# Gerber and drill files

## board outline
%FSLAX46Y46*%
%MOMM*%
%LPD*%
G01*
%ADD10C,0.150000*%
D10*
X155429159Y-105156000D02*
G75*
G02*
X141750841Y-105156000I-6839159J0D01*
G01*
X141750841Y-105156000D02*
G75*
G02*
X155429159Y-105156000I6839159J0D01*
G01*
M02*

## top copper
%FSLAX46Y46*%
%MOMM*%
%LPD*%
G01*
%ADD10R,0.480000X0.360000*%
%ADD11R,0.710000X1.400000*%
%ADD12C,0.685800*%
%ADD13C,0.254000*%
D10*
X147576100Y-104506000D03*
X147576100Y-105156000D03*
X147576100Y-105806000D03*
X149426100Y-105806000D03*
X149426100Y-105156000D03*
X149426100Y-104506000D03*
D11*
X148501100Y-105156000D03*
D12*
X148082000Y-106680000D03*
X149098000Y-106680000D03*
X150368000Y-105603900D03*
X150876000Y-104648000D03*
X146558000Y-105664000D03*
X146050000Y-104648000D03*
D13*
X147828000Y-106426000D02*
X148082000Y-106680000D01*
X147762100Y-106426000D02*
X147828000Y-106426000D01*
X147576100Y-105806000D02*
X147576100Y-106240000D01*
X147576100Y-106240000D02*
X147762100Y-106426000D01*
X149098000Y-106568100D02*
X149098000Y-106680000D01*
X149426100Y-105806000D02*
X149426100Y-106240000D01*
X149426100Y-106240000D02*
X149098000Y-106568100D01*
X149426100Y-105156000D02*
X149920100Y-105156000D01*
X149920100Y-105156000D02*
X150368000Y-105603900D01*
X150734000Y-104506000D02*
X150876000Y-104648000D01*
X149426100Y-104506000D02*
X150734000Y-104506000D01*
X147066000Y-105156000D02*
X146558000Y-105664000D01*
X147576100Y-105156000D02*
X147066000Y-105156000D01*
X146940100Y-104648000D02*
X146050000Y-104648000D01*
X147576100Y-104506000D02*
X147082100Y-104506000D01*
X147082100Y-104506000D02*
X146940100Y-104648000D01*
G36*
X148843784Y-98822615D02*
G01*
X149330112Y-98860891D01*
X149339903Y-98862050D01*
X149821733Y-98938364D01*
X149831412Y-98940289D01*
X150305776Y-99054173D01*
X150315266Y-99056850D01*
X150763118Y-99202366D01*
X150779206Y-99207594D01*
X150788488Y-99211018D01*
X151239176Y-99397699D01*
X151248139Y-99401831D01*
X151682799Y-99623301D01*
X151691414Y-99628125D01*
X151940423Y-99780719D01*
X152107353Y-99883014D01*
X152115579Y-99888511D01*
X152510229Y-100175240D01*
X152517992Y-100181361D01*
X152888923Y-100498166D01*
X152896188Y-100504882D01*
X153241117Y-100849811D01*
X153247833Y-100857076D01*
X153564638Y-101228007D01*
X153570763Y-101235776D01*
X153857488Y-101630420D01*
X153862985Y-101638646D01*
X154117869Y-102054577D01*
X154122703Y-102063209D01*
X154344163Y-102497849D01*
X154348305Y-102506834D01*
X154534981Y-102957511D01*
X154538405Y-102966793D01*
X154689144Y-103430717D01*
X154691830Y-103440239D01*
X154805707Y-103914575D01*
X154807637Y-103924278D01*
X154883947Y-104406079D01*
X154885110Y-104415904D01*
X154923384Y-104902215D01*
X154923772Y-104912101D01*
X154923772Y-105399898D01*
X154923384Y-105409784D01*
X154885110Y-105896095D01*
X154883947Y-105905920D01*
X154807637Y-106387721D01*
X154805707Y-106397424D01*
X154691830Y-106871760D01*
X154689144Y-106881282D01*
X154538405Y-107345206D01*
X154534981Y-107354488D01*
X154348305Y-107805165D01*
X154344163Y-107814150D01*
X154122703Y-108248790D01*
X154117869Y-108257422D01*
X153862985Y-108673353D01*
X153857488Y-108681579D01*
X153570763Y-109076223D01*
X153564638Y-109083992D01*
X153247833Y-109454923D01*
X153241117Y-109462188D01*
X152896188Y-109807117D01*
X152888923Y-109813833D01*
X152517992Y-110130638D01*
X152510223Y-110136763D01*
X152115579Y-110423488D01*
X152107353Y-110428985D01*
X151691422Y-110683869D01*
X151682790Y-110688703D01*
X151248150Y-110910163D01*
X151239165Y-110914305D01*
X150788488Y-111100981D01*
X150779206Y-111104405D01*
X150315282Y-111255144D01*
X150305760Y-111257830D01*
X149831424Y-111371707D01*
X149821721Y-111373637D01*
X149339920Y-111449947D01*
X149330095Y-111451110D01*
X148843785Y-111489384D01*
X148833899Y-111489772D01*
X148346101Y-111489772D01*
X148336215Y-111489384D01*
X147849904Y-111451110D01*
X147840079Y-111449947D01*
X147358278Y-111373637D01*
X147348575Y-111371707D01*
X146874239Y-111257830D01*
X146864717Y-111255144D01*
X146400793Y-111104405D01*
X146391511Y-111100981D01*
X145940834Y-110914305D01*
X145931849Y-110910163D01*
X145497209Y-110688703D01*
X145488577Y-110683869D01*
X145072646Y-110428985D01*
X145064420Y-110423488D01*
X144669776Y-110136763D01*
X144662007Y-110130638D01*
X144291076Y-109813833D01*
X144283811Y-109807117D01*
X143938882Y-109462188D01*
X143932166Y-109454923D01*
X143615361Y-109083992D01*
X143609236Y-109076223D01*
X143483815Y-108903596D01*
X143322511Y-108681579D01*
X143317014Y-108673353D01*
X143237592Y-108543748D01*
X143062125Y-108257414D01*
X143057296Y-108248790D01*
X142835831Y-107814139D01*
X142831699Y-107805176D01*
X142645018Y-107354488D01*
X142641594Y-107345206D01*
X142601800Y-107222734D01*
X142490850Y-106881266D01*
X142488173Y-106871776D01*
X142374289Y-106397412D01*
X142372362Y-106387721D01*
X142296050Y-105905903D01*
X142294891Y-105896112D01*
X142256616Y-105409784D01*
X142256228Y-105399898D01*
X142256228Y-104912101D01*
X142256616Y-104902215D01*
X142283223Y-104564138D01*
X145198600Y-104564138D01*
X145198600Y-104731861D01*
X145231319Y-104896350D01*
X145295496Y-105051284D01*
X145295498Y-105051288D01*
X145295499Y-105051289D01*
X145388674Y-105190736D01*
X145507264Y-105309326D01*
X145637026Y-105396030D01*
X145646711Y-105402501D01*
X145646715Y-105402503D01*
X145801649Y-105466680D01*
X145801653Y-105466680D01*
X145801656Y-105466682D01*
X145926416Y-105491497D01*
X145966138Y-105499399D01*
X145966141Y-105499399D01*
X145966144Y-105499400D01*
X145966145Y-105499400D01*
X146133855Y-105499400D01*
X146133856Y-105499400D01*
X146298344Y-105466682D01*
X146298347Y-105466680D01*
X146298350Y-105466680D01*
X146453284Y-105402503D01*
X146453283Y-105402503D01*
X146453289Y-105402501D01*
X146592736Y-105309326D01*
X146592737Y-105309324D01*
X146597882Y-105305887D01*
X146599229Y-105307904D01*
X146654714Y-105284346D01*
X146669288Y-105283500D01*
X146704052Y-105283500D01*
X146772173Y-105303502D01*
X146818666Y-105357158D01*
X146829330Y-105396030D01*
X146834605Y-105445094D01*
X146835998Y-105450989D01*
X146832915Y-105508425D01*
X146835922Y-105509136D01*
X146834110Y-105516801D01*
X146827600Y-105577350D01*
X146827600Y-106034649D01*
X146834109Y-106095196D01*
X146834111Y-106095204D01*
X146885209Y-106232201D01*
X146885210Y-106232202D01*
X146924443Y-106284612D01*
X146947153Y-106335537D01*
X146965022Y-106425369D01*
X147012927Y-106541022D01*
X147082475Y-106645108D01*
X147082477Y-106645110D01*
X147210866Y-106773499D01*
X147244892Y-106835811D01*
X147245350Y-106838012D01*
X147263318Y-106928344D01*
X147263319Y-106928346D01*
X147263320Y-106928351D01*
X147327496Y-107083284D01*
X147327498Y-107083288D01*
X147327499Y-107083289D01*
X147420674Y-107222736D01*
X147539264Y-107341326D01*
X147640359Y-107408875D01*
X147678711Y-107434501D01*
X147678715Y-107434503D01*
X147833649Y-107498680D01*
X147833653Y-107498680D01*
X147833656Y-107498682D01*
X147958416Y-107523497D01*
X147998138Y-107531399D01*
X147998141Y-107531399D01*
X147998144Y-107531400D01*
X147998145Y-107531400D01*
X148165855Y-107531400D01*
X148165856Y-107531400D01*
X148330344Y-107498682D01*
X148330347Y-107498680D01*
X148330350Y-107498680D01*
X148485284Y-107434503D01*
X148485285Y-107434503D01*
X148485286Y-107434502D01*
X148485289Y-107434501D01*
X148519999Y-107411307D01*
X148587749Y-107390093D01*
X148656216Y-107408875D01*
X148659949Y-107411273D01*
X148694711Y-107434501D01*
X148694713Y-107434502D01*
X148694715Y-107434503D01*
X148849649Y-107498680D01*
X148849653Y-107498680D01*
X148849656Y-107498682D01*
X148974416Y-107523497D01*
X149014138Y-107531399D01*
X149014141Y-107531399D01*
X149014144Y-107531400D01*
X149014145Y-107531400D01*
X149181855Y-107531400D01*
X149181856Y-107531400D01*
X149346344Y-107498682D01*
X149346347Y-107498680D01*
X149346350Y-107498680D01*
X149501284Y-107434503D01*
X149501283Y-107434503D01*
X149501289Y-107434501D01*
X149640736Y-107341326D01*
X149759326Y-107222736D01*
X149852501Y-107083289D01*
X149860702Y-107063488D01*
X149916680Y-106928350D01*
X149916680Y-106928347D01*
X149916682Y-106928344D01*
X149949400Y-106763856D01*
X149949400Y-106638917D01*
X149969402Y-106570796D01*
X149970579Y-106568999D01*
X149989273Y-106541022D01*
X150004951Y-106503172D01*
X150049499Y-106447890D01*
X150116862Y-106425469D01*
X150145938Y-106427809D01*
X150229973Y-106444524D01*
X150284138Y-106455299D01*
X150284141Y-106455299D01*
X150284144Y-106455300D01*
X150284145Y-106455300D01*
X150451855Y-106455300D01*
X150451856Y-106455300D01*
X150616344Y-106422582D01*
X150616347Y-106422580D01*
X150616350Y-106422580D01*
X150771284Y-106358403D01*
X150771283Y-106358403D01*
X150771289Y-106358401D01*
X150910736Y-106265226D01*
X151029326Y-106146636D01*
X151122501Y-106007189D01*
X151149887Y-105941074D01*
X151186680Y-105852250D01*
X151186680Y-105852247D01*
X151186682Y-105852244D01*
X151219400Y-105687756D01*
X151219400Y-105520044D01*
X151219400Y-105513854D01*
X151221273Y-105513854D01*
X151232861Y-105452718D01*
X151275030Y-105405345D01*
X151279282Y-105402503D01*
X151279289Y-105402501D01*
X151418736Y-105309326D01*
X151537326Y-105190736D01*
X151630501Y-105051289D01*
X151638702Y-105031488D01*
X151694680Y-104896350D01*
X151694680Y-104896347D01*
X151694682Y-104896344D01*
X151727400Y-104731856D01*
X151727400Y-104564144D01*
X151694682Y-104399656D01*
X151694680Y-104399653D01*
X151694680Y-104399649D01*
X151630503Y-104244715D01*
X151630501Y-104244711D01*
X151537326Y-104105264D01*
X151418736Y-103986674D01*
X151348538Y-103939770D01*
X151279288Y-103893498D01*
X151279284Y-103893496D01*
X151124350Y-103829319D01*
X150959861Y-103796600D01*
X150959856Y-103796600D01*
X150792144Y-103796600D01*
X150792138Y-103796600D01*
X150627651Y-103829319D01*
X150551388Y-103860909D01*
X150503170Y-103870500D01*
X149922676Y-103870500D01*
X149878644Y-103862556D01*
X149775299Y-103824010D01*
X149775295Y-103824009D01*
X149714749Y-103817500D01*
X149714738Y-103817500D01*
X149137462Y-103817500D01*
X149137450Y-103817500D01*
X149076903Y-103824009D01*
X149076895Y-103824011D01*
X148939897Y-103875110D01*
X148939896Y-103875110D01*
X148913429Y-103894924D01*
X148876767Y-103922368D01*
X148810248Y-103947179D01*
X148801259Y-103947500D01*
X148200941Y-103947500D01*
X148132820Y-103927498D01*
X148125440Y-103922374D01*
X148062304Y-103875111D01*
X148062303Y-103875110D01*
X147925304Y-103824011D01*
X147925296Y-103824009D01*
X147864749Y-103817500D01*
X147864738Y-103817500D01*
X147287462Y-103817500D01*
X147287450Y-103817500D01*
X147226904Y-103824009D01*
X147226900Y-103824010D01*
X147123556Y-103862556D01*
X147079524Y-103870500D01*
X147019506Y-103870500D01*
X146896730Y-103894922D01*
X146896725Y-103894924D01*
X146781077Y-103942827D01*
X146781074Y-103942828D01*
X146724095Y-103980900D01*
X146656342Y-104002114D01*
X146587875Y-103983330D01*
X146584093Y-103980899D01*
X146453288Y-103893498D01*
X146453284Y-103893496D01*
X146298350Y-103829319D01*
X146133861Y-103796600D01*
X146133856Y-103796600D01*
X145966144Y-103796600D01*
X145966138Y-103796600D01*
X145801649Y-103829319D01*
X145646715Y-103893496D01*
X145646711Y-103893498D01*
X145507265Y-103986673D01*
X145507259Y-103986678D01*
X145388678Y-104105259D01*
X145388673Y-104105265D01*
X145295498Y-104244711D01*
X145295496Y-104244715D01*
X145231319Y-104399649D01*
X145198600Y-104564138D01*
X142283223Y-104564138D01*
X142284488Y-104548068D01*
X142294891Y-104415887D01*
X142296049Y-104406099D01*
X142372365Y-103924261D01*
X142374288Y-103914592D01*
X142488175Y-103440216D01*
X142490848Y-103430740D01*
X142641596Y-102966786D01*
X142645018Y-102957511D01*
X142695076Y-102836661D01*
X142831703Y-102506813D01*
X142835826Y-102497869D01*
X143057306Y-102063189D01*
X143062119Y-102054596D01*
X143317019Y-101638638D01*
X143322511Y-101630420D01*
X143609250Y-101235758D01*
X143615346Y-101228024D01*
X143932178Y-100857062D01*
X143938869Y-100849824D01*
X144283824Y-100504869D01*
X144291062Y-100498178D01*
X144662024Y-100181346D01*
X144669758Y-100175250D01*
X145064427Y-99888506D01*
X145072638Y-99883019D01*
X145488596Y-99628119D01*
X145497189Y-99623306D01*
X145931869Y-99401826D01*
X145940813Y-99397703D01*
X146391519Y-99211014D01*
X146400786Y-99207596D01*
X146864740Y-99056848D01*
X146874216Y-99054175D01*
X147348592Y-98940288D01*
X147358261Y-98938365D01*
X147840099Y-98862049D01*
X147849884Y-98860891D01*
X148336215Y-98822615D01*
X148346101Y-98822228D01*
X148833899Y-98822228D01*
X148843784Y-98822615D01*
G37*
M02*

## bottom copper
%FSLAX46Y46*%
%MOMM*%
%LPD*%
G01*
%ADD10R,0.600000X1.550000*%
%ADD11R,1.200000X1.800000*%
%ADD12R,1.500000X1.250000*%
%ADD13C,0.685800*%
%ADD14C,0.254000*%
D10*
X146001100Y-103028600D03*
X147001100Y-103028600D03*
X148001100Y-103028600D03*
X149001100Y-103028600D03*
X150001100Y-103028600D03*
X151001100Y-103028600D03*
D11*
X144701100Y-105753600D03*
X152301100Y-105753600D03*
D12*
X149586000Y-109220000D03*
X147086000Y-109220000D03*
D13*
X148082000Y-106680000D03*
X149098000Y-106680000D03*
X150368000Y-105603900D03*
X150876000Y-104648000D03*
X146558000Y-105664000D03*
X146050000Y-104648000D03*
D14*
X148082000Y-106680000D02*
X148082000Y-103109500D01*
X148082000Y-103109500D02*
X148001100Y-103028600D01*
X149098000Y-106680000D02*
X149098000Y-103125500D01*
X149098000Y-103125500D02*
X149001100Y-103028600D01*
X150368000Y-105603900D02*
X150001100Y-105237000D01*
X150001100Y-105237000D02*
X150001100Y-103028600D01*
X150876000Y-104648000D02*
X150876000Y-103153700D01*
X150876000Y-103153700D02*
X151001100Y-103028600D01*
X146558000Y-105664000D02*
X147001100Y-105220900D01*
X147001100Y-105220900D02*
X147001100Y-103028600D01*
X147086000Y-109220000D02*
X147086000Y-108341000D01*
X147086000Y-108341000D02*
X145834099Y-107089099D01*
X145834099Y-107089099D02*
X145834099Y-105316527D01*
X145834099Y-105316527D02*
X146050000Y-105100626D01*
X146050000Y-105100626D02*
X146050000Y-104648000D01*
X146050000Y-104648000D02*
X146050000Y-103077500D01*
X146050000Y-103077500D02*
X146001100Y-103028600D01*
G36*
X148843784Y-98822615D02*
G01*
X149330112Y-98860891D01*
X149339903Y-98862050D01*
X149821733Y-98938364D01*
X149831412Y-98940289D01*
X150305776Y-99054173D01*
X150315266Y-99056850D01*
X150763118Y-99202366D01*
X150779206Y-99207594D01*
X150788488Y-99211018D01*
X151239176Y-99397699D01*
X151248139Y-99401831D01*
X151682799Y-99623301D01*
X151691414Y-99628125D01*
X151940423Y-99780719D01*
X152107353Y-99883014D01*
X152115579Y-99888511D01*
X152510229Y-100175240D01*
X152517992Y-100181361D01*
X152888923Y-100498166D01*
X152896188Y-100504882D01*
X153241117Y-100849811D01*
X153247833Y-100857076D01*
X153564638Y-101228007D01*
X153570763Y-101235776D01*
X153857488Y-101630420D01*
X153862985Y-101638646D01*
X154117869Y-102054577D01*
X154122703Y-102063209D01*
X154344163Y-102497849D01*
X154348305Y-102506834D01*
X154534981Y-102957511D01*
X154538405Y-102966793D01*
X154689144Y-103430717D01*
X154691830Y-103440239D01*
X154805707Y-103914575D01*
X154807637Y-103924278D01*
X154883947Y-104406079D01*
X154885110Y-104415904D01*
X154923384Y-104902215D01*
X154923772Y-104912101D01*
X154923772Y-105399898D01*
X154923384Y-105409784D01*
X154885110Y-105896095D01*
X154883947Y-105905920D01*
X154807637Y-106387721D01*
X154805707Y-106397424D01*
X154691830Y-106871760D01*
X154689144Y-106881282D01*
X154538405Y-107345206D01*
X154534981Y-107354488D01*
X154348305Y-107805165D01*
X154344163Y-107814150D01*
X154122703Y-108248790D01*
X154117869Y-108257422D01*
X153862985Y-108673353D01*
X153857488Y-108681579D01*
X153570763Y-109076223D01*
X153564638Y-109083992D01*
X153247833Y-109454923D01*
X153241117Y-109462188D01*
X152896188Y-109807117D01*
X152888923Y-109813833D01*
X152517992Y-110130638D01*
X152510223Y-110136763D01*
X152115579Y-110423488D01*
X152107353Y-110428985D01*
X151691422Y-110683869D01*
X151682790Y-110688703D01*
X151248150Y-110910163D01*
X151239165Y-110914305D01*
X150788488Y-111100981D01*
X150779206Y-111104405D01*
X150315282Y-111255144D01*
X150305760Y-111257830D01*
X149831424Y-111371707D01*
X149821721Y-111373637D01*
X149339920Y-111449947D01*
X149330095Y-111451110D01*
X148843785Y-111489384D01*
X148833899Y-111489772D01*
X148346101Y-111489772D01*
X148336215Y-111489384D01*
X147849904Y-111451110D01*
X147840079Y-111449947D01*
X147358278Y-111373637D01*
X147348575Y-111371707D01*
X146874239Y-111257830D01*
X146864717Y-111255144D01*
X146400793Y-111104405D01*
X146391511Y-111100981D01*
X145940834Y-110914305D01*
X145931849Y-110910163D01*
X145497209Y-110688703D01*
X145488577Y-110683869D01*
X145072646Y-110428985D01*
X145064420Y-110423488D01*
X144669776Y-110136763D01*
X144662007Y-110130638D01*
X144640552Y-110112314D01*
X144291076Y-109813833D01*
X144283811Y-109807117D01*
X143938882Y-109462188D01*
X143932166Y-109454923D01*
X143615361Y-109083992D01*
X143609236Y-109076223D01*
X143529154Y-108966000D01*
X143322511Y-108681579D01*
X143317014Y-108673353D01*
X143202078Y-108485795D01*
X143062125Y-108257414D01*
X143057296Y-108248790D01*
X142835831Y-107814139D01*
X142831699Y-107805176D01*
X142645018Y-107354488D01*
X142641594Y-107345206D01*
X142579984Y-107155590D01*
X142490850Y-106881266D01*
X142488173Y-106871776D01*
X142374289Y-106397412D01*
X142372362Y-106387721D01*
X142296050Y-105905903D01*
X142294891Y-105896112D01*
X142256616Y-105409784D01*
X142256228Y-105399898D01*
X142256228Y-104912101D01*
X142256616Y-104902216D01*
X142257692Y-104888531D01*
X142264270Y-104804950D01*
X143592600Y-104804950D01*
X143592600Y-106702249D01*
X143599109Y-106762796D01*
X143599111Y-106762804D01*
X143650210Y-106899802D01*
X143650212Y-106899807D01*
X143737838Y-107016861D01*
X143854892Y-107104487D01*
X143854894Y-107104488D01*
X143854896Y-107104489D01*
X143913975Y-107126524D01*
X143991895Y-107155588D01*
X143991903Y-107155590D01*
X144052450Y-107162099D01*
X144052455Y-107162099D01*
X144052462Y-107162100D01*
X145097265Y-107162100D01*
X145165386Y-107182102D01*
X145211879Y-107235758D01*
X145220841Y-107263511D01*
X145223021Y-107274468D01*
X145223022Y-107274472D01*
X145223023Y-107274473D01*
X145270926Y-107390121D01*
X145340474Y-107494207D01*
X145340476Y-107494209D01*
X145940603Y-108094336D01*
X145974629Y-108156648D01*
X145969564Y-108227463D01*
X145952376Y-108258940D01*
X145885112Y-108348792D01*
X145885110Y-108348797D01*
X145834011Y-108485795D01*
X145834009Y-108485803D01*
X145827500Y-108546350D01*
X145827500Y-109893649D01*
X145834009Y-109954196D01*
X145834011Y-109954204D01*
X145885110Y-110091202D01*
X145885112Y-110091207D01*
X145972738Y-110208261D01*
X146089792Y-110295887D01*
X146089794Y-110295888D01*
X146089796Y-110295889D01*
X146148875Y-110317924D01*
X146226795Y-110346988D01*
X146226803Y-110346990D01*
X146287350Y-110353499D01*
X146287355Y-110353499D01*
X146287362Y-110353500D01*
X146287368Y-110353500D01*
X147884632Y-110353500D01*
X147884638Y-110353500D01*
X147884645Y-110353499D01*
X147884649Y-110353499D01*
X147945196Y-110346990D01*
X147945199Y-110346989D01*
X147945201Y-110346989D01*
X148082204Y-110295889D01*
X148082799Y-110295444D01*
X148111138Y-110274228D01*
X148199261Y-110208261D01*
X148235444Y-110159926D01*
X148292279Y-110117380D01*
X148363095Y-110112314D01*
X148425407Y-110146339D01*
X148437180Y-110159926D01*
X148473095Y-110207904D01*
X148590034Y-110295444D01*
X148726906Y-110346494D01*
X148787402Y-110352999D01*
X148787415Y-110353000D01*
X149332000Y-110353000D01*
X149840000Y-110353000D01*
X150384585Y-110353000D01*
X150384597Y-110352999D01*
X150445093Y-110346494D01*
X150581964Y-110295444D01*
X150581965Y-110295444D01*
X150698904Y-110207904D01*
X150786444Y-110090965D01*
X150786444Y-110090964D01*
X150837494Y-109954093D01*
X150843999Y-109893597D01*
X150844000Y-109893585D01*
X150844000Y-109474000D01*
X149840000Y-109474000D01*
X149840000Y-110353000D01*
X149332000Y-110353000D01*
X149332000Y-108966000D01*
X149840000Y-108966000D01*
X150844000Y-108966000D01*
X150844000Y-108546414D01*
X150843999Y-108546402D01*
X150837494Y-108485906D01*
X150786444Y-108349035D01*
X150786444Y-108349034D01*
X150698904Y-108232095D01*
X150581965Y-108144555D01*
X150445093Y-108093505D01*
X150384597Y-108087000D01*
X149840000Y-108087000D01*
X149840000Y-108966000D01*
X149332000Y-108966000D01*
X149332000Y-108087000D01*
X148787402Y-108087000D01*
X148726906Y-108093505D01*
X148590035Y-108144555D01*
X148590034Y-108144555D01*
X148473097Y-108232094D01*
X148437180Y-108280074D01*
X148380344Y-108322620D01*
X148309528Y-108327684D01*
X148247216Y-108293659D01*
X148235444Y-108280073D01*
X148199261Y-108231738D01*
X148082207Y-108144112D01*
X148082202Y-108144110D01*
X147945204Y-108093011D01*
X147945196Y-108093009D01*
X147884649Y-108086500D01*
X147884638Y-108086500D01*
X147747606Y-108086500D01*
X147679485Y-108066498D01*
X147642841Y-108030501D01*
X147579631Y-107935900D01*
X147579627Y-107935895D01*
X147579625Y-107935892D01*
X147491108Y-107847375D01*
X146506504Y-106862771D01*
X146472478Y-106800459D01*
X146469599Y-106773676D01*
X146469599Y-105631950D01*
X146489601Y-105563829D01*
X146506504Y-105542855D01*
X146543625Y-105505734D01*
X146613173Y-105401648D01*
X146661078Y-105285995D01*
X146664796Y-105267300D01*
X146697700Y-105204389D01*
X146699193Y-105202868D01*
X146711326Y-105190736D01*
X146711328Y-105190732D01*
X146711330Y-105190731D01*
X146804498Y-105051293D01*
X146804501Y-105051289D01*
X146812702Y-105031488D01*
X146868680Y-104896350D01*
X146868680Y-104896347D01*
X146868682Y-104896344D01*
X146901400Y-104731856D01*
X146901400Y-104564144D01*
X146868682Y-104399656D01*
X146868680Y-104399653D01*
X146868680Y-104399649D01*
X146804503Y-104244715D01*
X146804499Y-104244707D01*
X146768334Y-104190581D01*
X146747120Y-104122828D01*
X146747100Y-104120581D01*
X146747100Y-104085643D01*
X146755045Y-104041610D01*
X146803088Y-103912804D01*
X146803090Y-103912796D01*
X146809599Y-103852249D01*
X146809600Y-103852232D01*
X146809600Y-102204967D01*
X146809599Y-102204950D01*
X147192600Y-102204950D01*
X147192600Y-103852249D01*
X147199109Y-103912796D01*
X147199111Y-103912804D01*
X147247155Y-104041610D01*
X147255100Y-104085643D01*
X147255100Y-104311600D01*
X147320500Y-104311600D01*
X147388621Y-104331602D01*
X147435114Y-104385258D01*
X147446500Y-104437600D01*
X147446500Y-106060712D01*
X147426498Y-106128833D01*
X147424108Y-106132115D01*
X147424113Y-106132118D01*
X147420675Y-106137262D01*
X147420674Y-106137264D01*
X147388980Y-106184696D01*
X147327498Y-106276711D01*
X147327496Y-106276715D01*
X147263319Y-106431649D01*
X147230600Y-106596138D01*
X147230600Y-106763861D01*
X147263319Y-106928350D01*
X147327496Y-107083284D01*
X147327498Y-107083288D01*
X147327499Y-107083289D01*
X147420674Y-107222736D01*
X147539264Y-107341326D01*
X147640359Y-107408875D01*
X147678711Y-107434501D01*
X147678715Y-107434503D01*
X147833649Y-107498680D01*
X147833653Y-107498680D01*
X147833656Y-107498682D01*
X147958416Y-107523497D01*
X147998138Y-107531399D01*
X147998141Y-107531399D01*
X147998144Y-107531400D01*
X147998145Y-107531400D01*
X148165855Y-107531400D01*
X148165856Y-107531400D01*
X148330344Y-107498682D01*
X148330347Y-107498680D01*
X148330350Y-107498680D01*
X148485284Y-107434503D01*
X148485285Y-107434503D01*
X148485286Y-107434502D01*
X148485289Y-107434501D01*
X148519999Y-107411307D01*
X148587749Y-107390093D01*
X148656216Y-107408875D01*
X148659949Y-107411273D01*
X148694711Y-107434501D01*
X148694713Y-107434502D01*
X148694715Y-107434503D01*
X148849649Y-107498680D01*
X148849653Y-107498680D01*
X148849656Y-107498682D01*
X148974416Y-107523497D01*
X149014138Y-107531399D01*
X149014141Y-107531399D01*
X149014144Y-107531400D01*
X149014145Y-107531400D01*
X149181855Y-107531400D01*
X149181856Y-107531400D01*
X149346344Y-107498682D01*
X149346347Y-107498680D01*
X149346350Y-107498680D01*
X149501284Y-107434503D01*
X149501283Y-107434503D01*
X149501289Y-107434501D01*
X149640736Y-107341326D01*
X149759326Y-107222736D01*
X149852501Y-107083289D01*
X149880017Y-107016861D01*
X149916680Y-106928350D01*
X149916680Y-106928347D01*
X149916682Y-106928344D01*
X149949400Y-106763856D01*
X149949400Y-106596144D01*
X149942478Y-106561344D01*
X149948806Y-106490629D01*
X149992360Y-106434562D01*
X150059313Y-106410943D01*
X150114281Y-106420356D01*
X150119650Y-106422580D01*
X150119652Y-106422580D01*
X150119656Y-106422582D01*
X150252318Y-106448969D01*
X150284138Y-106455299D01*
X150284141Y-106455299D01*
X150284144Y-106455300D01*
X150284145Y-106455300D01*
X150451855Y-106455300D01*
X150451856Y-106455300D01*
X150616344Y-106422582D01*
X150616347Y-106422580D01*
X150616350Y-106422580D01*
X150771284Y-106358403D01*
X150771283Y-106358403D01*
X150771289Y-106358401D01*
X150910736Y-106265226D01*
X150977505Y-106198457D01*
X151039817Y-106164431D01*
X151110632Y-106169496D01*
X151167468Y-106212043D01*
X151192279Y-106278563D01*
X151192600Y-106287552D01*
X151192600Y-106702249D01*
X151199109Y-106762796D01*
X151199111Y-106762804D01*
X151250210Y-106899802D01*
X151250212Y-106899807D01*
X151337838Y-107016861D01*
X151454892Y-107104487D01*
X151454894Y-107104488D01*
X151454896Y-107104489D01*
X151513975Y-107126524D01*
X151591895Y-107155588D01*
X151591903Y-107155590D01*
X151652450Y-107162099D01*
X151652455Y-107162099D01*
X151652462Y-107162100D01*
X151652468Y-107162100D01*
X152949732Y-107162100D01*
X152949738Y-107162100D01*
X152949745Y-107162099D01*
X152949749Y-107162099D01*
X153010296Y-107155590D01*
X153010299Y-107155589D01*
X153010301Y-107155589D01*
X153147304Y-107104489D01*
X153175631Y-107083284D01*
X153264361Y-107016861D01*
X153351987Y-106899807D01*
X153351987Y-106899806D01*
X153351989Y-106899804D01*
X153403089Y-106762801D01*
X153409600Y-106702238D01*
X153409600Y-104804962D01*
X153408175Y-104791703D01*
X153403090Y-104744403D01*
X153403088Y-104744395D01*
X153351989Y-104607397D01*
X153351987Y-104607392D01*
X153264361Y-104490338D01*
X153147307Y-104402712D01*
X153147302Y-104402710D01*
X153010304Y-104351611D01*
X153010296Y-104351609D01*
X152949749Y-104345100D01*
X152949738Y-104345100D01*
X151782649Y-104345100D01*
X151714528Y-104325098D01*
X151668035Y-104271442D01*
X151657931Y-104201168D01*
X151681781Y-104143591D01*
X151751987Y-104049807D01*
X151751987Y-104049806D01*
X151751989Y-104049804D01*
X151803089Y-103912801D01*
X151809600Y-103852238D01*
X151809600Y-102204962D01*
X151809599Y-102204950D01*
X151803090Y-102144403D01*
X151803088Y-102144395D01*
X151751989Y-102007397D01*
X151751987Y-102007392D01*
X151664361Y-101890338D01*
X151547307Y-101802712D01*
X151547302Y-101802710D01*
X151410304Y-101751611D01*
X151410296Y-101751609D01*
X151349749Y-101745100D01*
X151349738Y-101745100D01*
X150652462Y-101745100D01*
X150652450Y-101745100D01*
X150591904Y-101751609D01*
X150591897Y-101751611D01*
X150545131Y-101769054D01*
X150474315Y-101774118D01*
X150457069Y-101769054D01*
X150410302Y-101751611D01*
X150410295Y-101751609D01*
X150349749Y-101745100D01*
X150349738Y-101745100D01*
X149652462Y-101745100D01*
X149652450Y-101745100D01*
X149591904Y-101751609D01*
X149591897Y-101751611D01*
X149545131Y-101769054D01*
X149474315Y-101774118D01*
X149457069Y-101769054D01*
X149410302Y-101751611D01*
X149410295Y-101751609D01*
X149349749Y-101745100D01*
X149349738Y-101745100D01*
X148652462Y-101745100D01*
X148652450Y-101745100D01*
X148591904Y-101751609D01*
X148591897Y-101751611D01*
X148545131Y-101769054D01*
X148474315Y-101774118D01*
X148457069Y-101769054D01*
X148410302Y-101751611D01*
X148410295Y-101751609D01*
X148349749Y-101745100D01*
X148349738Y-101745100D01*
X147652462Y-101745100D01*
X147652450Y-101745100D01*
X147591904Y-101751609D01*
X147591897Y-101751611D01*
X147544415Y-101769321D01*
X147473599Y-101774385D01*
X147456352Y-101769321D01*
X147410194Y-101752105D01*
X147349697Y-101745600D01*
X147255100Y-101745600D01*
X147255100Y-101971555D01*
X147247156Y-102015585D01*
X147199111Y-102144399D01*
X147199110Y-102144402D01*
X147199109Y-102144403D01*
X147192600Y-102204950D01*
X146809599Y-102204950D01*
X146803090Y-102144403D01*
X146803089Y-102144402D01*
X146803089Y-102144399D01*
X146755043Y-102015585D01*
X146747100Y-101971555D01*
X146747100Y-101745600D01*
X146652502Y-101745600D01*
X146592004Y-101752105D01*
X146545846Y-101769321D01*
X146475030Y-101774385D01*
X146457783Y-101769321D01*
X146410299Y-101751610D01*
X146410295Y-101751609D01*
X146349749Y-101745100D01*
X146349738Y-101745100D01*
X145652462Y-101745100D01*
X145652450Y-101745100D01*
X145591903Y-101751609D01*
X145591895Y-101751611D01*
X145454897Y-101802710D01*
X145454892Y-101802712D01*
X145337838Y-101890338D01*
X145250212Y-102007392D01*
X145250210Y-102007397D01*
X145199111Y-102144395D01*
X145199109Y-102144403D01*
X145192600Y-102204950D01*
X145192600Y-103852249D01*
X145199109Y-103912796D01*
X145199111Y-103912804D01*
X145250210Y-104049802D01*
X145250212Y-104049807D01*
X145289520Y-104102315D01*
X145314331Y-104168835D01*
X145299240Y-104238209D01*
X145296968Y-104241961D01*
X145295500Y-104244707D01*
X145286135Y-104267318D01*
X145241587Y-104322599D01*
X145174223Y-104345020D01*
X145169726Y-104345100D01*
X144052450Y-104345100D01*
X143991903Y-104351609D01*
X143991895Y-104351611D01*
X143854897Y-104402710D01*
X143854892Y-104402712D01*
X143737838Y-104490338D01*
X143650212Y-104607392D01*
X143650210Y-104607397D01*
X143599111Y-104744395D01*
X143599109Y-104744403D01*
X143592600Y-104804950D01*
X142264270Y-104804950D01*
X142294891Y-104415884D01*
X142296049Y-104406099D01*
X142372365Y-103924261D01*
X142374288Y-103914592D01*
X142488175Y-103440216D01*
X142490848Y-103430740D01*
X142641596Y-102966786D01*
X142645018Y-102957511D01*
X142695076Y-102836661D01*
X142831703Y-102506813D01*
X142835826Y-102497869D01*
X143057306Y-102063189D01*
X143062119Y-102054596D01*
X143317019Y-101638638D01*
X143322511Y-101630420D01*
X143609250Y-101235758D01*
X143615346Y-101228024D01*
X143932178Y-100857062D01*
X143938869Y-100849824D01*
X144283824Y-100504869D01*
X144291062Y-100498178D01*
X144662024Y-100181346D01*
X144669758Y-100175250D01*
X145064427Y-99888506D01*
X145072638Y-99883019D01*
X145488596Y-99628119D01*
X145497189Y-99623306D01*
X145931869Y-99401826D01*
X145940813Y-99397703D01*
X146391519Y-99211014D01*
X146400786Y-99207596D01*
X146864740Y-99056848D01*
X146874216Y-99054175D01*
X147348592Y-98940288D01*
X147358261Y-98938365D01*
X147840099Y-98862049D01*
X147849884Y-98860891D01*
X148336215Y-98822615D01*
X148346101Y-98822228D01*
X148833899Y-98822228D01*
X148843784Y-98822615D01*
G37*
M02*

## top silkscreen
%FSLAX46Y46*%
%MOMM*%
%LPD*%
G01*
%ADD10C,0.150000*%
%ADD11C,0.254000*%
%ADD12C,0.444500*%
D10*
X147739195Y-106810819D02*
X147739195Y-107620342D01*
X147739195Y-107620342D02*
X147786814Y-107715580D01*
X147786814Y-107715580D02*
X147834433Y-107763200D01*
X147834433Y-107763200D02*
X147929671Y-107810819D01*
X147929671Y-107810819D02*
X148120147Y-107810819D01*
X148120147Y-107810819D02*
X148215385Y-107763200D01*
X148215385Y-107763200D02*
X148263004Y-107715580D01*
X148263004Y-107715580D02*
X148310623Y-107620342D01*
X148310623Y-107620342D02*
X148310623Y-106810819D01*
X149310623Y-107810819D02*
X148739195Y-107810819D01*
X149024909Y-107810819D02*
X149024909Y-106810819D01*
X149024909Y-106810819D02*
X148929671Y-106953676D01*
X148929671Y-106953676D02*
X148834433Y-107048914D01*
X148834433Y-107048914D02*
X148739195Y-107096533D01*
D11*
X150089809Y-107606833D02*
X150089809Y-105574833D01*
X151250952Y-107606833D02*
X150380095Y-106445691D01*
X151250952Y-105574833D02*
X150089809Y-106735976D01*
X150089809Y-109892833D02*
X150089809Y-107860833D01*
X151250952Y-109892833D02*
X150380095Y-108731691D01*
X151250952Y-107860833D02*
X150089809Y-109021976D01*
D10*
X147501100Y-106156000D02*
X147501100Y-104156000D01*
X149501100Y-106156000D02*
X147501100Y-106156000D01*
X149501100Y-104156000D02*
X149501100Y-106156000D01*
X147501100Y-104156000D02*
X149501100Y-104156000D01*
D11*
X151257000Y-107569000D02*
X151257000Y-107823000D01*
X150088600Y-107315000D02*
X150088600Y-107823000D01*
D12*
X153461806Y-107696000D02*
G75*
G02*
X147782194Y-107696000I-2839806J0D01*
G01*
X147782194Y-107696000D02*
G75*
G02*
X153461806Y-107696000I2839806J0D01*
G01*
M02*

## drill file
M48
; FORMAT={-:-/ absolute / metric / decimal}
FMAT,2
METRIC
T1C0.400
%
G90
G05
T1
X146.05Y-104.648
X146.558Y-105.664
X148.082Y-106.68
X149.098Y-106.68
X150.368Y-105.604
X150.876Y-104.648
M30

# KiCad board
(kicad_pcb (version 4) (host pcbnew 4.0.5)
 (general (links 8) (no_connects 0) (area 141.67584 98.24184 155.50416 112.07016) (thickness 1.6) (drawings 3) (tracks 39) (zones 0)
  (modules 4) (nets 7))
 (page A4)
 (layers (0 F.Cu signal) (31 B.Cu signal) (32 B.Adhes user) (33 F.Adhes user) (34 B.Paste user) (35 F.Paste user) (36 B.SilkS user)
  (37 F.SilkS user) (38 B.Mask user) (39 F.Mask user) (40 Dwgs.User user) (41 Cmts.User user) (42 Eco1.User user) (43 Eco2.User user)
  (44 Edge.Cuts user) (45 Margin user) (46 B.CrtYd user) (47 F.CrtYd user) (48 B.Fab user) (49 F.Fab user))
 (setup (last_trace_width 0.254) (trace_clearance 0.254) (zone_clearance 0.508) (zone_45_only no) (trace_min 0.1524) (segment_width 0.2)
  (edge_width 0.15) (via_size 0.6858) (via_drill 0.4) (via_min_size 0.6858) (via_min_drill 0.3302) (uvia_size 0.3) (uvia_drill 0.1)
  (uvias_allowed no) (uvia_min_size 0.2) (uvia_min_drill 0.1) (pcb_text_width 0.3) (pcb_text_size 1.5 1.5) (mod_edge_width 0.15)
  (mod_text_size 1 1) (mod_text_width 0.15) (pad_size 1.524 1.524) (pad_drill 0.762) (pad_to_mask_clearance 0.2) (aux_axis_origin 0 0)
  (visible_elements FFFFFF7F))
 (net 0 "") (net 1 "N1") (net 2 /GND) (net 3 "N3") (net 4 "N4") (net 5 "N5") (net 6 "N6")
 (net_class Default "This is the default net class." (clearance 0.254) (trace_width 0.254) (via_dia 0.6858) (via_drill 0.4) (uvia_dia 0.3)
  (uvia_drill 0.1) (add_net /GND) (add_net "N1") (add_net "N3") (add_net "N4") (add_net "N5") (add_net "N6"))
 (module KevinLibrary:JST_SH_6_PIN (layer B.Cu) (at 148.5011 105.0036)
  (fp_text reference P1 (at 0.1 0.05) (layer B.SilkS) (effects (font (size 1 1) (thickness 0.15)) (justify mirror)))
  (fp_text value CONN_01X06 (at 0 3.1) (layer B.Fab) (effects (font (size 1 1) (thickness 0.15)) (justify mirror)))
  (pad 1 smd rect (at -2.5 -1.975) (size 0.6 1.55) (layers B.Cu B.Paste B.Mask) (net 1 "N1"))
  (pad 2 smd rect (at -1.5 -1.975) (size 0.6 1.55) (layers B.Cu B.Paste B.Mask) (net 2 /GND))
  (pad 3 smd rect (at -0.5 -1.975) (size 0.6 1.55) (layers B.Cu B.Paste B.Mask) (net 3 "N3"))
  (pad 4 smd rect (at 0.5 -1.975) (size 0.6 1.55) (layers B.Cu B.Paste B.Mask) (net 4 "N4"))
  (pad 5 smd rect (at 1.5 -1.975) (size 0.6 1.55) (layers B.Cu B.Paste B.Mask) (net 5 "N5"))
  (pad 6 smd rect (at 2.5 -1.975) (size 0.6 1.55) (layers B.Cu B.Paste B.Mask) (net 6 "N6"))
  (pad "" smd rect (at -3.8 0.75) (size 1.2 1.8) (layers B.Cu B.Paste B.Mask))
  (pad "" smd rect (at 3.8 0.75) (size 1.2 1.8) (layers B.Cu B.Paste B.Mask)))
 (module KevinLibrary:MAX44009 (layer F.Cu) (at 148.5011 105.156)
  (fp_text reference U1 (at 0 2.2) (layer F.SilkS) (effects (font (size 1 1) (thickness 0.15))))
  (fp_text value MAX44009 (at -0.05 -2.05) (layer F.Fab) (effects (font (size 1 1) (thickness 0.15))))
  (fp_line (start -1 1) (end -1 -1) (layer F.SilkS) (width 0.15))
  (fp_line (start 1 1) (end -1 1) (layer F.SilkS) (width 0.15))
  (fp_line (start 1 -1) (end 1 1) (layer F.SilkS) (width 0.15))
  (fp_line (start -1 -1) (end 1 -1) (layer F.SilkS) (width 0.15))
  (pad 1 smd rect (at -0.925 -0.65) (size 0.48 0.36) (layers F.Cu F.Paste F.Mask) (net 1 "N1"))
  (pad 2 smd rect (at -0.925 0) (size 0.48 0.36) (layers F.Cu F.Paste F.Mask) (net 2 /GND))
  (pad 3 smd rect (at -0.925 0.65) (size 0.48 0.36) (layers F.Cu F.Paste F.Mask) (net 3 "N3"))
  (pad 4 smd rect (at 0.925 0.65) (size 0.48 0.36) (layers F.Cu F.Paste F.Mask) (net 4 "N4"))
  (pad 5 smd rect (at 0.925 0) (size 0.48 0.36) (layers F.Cu F.Paste F.Mask) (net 5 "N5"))
  (pad 6 smd rect (at 0.925 -0.65) (size 0.48 0.36) (layers F.Cu F.Paste F.Mask) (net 6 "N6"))
  (pad "" smd rect (at 0 0) (size 0.71 1.4) (layers F.Cu F.Paste F.Mask)))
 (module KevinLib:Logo (layer F.Cu) (at 150.622 107.696)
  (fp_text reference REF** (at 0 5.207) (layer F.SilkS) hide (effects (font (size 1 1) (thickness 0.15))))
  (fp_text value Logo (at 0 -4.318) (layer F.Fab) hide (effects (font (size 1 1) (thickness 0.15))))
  (fp_line (start 0.635 -0.127) (end 0.635 0.127) (layer F.SilkS) (width 0.254))
  (fp_line (start -0.5334 -0.381) (end -0.5334 0.127) (layer F.SilkS) (width 0.254))
  (fp_circle (center 0 0) (end 2.54 -1.27) (layer F.SilkS) (width 0.4445))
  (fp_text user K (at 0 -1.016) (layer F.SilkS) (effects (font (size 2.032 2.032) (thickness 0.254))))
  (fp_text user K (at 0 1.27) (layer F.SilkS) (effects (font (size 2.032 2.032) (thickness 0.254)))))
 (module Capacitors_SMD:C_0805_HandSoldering (layer B.Cu) (at 148.336 109.22 180)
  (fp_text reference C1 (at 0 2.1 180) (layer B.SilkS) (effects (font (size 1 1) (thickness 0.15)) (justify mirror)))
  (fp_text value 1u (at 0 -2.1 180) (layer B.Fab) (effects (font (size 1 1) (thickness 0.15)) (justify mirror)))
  (pad 1 smd rect (at -1.25 0 180) (size 1.5 1.25) (layers B.Cu B.Paste B.Mask) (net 2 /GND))
  (pad 2 smd rect (at 1.25 0 180) (size 1.5 1.25) (layers B.Cu B.Paste B.Mask) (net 1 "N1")))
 (gr_circle (center 148.59 105.156) (end 154.94 102.616) (layer Edge.Cuts) (width 0.15))
 (segment (start 148.082 106.68) (end 148.082 103.1095) (width 0.254) (layer B.Cu) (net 3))
 (segment (start 148.082 103.1095) (end 148.0011 103.0286) (width 0.254) (layer B.Cu) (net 3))
 (segment (start 147.828 106.426) (end 148.082 106.68) (width 0.254) (layer F.Cu) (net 3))
 (via (at 148.082 106.68) (size 0.6858) (drill 0.4) (layers F.Cu B.Cu) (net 3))
 (segment (start 147.7621 106.426) (end 147.828 106.426) (width 0.254) (layer F.Cu) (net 3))
 (segment (start 147.5761 105.806) (end 147.5761 106.24) (width 0.254) (layer F.Cu) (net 3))
 (segment (start 147.5761 106.24) (end 147.7621 106.426) (width 0.254) (layer F.Cu) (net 3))
 (segment (start 149.098 106.68) (end 149.098 103.1255) (width 0.254) (layer B.Cu) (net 4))
 (segment (start 149.098 103.1255) (end 149.0011 103.0286) (width 0.254) (layer B.Cu) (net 4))
 (segment (start 149.098 106.5681) (end 149.098 106.68) (width 0.254) (layer F.Cu) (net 4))
 (via (at 149.098 106.68) (size 0.6858) (drill 0.4) (layers F.Cu B.Cu) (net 4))
 (segment (start 149.4261 105.806) (end 149.4261 106.24) (width 0.254) (layer F.Cu) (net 4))
 (segment (start 149.4261 106.24) (end 149.098 106.5681) (width 0.254) (layer F.Cu) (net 4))
 (segment (start 150.368 105.6039) (end 150.0011 105.237) (width 0.254) (layer B.Cu) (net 5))
 (segment (start 150.0011 105.237) (end 150.0011 103.0286) (width 0.254) (layer B.Cu) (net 5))
 (via (at 150.368 105.6039) (size 0.6858) (drill 0.4) (layers F.Cu B.Cu) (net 5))
 (segment (start 149.4261 105.156) (end 149.9201 105.156) (width 0.254) (layer F.Cu) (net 5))
 (segment (start 149.9201 105.156) (end 150.368 105.6039) (width 0.254) (layer F.Cu) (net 5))
 (segment (start 150.876 104.648) (end 150.876 103.1537) (width 0.254) (layer B.Cu) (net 6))
 (segment (start 150.876 103.1537) (end 151.0011 103.0286) (width 0.254) (layer B.Cu) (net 6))
 (segment (start 150.734 104.506) (end 150.876 104.648) (width 0.254) (layer F.Cu) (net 6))
 (via (at 150.876 104.648) (size 0.6858) (drill 0.4) (layers F.Cu B.Cu) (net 6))
 (segment (start 149.4261 104.506) (end 150.734 104.506) (width 0.254) (layer F.Cu) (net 6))
 (segment (start 146.558 105.664) (end 147.0011 105.2209) (width 0.254) (layer B.Cu) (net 2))
 (segment (start 147.0011 105.2209) (end 147.0011 103.0286) (width 0.254) (layer B.Cu) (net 2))
 (segment (start 147.066 105.156) (end 146.558 105.664) (width 0.254) (layer F.Cu) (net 2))
 (via (at 146.558 105.664) (size 0.6858) (drill 0.4) (layers F.Cu B.Cu) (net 2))
 (segment (start 147.5761 105.156) (end 147.066 105.156) (width 0.254) (layer F.Cu) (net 2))
 (segment (start 147.086 109.22) (end 147.086 108.341) (width 0.254) (layer B.Cu) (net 1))
 (segment (start 147.086 108.341) (end 145.834099 107.089099) (width 0.254) (layer B.Cu) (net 1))
 (segment (start 145.834099 107.089099) (end 145.834099 105.316527) (width 0.254) (layer B.Cu) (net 1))
 (segment (start 145.834099 105.316527) (end 146.05 105.100626) (width 0.254) (layer B.Cu) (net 1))
 (segment (start 146.05 105.100626) (end 146.05 104.648) (width 0.254) (layer B.Cu) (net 1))
 (segment (start 146.05 104.648) (end 146.05 103.0775) (width 0.254) (layer B.Cu) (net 1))
 (segment (start 146.05 103.0775) (end 146.0011 103.0286) (width 0.254) (layer B.Cu) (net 1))
 (segment (start 146.9401 104.648) (end 146.05 104.648) (width 0.254) (layer F.Cu) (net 1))
 (via (at 146.05 104.648) (size 0.6858) (drill 0.4) (layers F.Cu B.Cu) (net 1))
 (segment (start 147.5761 104.506) (end 147.0821 104.506) (width 0.254) (layer F.Cu) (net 1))
 (segment (start 147.0821 104.506) (end 146.9401 104.648) (width 0.254) (layer F.Cu) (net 1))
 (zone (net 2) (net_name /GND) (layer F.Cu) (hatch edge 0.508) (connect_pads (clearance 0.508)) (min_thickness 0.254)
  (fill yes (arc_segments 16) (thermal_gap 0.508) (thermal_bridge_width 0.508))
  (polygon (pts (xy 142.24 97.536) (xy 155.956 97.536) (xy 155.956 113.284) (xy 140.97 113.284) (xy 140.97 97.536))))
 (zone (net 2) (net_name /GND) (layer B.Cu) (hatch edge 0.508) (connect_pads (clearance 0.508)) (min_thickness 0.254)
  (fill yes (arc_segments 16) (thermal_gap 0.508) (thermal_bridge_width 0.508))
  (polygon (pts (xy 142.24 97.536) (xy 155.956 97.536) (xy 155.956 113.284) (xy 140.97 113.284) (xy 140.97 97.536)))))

